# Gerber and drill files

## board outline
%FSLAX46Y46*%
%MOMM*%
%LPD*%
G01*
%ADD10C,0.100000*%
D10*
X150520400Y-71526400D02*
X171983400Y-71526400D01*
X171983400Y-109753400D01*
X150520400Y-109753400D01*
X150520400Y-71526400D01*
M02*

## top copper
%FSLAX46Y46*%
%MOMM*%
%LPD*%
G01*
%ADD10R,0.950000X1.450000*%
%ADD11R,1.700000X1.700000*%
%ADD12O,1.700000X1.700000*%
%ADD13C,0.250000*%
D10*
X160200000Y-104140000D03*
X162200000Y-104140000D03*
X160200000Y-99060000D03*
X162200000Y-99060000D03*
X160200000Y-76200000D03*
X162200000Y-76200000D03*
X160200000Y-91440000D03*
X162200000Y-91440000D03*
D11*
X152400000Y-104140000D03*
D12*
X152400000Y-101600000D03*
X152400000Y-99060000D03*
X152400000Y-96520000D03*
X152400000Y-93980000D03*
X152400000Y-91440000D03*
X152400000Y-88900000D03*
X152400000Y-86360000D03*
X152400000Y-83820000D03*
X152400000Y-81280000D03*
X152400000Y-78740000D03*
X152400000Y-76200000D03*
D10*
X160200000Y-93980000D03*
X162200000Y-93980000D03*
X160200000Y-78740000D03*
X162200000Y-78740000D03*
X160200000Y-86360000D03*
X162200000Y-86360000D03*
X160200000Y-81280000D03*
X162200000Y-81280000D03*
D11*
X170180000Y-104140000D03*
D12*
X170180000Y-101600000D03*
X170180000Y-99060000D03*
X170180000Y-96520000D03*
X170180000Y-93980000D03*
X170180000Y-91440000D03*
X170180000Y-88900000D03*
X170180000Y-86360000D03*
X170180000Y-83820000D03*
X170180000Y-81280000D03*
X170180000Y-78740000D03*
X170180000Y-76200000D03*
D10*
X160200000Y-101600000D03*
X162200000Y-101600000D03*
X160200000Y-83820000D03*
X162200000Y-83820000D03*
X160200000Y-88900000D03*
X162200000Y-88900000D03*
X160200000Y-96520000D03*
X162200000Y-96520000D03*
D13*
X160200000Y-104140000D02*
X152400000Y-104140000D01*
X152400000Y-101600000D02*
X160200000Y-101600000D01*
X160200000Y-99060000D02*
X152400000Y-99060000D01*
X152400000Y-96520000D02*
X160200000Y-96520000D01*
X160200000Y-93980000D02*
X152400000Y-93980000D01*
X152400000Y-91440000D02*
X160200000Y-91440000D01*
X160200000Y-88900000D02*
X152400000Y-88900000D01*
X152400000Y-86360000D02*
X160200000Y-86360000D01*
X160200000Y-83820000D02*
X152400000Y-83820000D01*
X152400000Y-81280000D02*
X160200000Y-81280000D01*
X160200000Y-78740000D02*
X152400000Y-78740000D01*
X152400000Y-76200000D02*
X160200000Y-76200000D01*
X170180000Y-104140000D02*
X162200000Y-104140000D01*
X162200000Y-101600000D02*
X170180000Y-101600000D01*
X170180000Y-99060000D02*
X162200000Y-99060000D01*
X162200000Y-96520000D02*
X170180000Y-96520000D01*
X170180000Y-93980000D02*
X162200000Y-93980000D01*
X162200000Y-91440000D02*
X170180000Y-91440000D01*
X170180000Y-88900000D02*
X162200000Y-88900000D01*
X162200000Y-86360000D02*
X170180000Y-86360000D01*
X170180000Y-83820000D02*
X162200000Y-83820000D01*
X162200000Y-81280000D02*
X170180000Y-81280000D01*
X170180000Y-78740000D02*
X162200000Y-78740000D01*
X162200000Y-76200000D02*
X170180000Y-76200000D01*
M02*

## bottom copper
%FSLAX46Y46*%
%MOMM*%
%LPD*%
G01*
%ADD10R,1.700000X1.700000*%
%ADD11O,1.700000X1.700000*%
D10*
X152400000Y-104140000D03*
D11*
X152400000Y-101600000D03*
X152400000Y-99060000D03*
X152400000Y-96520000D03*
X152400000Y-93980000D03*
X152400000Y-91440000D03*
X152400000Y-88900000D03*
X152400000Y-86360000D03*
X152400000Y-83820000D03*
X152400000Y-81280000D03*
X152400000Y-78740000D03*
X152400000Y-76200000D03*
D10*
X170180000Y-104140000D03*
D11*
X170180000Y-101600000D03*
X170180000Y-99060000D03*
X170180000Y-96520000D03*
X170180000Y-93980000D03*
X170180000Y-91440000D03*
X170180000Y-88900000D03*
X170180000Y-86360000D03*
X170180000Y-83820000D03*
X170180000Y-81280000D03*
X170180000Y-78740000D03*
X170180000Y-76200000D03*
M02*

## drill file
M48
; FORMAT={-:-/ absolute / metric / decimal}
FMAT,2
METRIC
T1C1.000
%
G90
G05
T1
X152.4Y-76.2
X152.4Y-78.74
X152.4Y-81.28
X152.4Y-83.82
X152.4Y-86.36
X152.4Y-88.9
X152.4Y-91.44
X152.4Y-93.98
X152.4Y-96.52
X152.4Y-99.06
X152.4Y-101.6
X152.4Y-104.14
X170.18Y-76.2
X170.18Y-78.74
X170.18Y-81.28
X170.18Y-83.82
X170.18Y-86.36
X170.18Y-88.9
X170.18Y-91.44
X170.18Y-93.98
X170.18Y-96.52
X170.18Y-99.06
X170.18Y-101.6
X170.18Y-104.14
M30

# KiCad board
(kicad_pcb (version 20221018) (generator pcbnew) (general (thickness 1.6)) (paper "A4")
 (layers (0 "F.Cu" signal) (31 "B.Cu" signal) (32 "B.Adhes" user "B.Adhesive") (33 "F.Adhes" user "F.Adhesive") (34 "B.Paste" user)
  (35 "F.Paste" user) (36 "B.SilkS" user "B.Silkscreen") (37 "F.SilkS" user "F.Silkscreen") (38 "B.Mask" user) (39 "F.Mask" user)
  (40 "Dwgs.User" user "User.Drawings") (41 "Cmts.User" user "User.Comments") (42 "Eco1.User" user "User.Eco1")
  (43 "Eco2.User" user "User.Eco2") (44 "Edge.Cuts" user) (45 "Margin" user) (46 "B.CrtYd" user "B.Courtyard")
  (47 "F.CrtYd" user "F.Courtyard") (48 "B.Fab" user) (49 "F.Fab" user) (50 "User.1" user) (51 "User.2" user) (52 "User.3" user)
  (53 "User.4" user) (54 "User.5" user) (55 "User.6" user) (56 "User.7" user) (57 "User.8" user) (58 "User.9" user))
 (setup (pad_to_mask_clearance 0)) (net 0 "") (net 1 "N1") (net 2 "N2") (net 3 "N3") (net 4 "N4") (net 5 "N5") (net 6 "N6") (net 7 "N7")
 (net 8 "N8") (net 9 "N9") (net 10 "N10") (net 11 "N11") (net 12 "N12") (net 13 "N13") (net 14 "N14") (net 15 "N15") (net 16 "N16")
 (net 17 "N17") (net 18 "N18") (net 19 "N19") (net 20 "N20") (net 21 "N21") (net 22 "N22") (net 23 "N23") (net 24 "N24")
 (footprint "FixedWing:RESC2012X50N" (layer "F.Cu") (at 161.2 104.14)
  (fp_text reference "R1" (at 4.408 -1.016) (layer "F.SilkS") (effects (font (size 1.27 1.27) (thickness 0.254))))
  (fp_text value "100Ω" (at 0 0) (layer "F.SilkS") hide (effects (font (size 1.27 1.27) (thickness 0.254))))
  (pad "1" smd rect (at -1 0) (size 0.95 1.45) (layers "F.Cu" "F.Paste" "F.Mask") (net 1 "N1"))
  (pad "2" smd rect (at 1 0) (size 0.95 1.45) (layers "F.Cu" "F.Paste" "F.Mask") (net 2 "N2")))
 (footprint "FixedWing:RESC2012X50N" (layer "F.Cu") (at 161.2 99.06)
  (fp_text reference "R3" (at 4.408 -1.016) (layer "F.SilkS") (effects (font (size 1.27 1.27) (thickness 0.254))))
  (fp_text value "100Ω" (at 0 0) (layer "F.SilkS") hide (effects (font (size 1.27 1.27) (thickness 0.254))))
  (pad "1" smd rect (at -1 0) (size 0.95 1.45) (layers "F.Cu" "F.Paste" "F.Mask") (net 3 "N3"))
  (pad "2" smd rect (at 1 0) (size 0.95 1.45) (layers "F.Cu" "F.Paste" "F.Mask") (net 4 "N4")))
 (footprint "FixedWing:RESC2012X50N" (layer "F.Cu") (at 161.2 76.2)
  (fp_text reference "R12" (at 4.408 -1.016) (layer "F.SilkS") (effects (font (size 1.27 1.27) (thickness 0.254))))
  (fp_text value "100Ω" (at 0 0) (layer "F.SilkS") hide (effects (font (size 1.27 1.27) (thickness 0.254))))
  (pad "1" smd rect (at -1 0) (size 0.95 1.45) (layers "F.Cu" "F.Paste" "F.Mask") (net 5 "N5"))
  (pad "2" smd rect (at 1 0) (size 0.95 1.45) (layers "F.Cu" "F.Paste" "F.Mask") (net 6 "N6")))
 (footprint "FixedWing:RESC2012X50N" (layer "F.Cu") (at 161.2 91.44)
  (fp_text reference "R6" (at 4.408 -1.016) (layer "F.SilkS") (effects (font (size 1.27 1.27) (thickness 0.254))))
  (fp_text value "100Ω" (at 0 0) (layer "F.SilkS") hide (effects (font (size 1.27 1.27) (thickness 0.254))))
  (pad "1" smd rect (at -1 0) (size 0.95 1.45) (layers "F.Cu" "F.Paste" "F.Mask") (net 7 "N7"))
  (pad "2" smd rect (at 1 0) (size 0.95 1.45) (layers "F.Cu" "F.Paste" "F.Mask") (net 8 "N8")))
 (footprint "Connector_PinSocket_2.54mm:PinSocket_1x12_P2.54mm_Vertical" (layer "F.Cu") (at 152.4 104.14 180)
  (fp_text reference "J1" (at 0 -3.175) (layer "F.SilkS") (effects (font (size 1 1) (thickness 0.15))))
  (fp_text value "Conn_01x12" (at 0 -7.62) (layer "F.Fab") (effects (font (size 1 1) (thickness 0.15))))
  (pad "1" thru_hole rect (at 0 0 180) (size 1.7 1.7) (drill 1) (layers "*.Cu" "*.Mask") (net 1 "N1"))
  (pad "2" thru_hole oval (at 0 2.54 180) (size 1.7 1.7) (drill 1) (layers "*.Cu" "*.Mask") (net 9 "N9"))
  (pad "3" thru_hole oval (at 0 5.08 180) (size 1.7 1.7) (drill 1) (layers "*.Cu" "*.Mask") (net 3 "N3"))
  (pad "4" thru_hole oval (at 0 7.62 180) (size 1.7 1.7) (drill 1) (layers "*.Cu" "*.Mask") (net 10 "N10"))
  (pad "5" thru_hole oval (at 0 10.16 180) (size 1.7 1.7) (drill 1) (layers "*.Cu" "*.Mask") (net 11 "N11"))
  (pad "6" thru_hole oval (at 0 12.7 180) (size 1.7 1.7) (drill 1) (layers "*.Cu" "*.Mask") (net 7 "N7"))
  (pad "7" thru_hole oval (at 0 15.24 180) (size 1.7 1.7) (drill 1) (layers "*.Cu" "*.Mask") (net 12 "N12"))
  (pad "8" thru_hole oval (at 0 17.78 180) (size 1.7 1.7) (drill 1) (layers "*.Cu" "*.Mask") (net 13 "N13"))
  (pad "9" thru_hole oval (at 0 20.32 180) (size 1.7 1.7) (drill 1) (layers "*.Cu" "*.Mask") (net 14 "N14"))
  (pad "10" thru_hole oval (at 0 22.86 180) (size 1.7 1.7) (drill 1) (layers "*.Cu" "*.Mask") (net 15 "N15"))
  (pad "11" thru_hole oval (at 0 25.4 180) (size 1.7 1.7) (drill 1) (layers "*.Cu" "*.Mask") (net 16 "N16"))
  (pad "12" thru_hole oval (at 0 27.94 180) (size 1.7 1.7) (drill 1) (layers "*.Cu" "*.Mask") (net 5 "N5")))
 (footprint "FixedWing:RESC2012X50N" (layer "F.Cu") (at 161.2 93.98)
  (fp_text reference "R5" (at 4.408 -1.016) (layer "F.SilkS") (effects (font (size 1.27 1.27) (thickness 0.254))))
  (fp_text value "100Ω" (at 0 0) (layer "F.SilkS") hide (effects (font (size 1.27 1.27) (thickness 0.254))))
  (pad "1" smd rect (at -1 0) (size 0.95 1.45) (layers "F.Cu" "F.Paste" "F.Mask") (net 11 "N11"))
  (pad "2" smd rect (at 1 0) (size 0.95 1.45) (layers "F.Cu" "F.Paste" "F.Mask") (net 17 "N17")))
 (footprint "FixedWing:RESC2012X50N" (layer "F.Cu") (at 161.2 78.74)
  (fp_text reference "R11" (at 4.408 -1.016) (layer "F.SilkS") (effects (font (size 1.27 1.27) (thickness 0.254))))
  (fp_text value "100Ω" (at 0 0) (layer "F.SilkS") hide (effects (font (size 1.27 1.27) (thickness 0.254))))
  (pad "1" smd rect (at -1 0) (size 0.95 1.45) (layers "F.Cu" "F.Paste" "F.Mask") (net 16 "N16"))
  (pad "2" smd rect (at 1 0) (size 0.95 1.45) (layers "F.Cu" "F.Paste" "F.Mask") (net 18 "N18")))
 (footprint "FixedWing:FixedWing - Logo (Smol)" (layer "F.Cu") (at 161.250214 73.970419)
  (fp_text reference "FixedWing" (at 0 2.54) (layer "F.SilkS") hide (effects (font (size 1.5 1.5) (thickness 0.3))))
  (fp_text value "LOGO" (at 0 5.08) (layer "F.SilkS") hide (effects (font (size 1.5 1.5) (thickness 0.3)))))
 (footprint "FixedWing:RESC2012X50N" (layer "F.Cu") (at 161.2 86.36)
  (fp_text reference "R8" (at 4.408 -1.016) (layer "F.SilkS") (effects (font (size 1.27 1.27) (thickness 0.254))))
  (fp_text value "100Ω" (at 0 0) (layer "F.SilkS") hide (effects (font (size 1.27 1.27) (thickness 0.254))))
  (pad "1" smd rect (at -1 0) (size 0.95 1.45) (layers "F.Cu" "F.Paste" "F.Mask") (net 13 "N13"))
  (pad "2" smd rect (at 1 0) (size 0.95 1.45) (layers "F.Cu" "F.Paste" "F.Mask") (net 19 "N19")))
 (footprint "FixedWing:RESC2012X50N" (layer "F.Cu") (at 161.2 81.28)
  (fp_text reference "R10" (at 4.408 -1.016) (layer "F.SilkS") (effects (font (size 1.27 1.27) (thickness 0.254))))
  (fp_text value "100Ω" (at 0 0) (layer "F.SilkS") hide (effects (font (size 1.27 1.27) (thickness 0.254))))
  (pad "1" smd rect (at -1 0) (size 0.95 1.45) (layers "F.Cu" "F.Paste" "F.Mask") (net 15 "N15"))
  (pad "2" smd rect (at 1 0) (size 0.95 1.45) (layers "F.Cu" "F.Paste" "F.Mask") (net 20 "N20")))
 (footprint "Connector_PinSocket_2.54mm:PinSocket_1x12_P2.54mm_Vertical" (layer "F.Cu") (at 170.18 104.14 180)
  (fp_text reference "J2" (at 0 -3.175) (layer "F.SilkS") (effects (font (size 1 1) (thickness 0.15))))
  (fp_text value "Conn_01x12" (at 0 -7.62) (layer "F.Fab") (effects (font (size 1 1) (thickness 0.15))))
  (pad "1" thru_hole rect (at 0 0 180) (size 1.7 1.7) (drill 1) (layers "*.Cu" "*.Mask") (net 2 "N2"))
  (pad "2" thru_hole oval (at 0 2.54 180) (size 1.7 1.7) (drill 1) (layers "*.Cu" "*.Mask") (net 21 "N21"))
  (pad "3" thru_hole oval (at 0 5.08 180) (size 1.7 1.7) (drill 1) (layers "*.Cu" "*.Mask") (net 4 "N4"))
  (pad "4" thru_hole oval (at 0 7.62 180) (size 1.7 1.7) (drill 1) (layers "*.Cu" "*.Mask") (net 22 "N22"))
  (pad "5" thru_hole oval (at 0 10.16 180) (size 1.7 1.7) (drill 1) (layers "*.Cu" "*.Mask") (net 17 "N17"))
  (pad "6" thru_hole oval (at 0 12.7 180) (size 1.7 1.7) (drill 1) (layers "*.Cu" "*.Mask") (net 8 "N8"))
  (pad "7" thru_hole oval (at 0 15.24 180) (size 1.7 1.7) (drill 1) (layers "*.Cu" "*.Mask") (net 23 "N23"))
  (pad "8" thru_hole oval (at 0 17.78 180) (size 1.7 1.7) (drill 1) (layers "*.Cu" "*.Mask") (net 19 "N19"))
  (pad "9" thru_hole oval (at 0 20.32 180) (size 1.7 1.7) (drill 1) (layers "*.Cu" "*.Mask") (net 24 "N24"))
  (pad "10" thru_hole oval (at 0 22.86 180) (size 1.7 1.7) (drill 1) (layers "*.Cu" "*.Mask") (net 20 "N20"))
  (pad "11" thru_hole oval (at 0 25.4 180) (size 1.7 1.7) (drill 1) (layers "*.Cu" "*.Mask") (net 18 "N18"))
  (pad "12" thru_hole oval (at 0 27.94 180) (size 1.7 1.7) (drill 1) (layers "*.Cu" "*.Mask") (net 6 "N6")))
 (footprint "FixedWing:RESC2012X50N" (layer "F.Cu") (at 161.2 101.6)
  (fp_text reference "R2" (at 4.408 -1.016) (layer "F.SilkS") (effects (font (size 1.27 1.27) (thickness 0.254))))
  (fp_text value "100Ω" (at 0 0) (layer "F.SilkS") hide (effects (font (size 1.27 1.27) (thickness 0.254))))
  (pad "1" smd rect (at -1 0) (size 0.95 1.45) (layers "F.Cu" "F.Paste" "F.Mask") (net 9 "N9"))
  (pad "2" smd rect (at 1 0) (size 0.95 1.45) (layers "F.Cu" "F.Paste" "F.Mask") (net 21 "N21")))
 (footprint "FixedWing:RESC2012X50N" (layer "F.Cu") (at 161.2 83.82)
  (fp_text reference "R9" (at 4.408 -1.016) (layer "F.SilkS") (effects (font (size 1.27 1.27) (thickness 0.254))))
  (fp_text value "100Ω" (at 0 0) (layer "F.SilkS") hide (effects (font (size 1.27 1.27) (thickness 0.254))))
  (pad "1" smd rect (at -1 0) (size 0.95 1.45) (layers "F.Cu" "F.Paste" "F.Mask") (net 14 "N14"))
  (pad "2" smd rect (at 1 0) (size 0.95 1.45) (layers "F.Cu" "F.Paste" "F.Mask") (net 24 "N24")))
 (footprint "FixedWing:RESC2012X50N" (layer "F.Cu") (at 161.2 88.9)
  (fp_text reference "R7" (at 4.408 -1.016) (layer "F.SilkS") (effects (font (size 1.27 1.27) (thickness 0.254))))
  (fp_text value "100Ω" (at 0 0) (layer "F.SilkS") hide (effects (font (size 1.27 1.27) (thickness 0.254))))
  (pad "1" smd rect (at -1 0) (size 0.95 1.45) (layers "F.Cu" "F.Paste" "F.Mask") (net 12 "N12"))
  (pad "2" smd rect (at 1 0) (size 0.95 1.45) (layers "F.Cu" "F.Paste" "F.Mask") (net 23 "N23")))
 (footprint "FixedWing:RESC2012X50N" (layer "F.Cu") (at 161.2 96.52)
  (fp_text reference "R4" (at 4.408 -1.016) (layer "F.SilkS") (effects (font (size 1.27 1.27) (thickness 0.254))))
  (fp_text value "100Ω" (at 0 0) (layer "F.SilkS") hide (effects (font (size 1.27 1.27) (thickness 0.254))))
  (pad "1" smd rect (at -1 0) (size 0.95 1.45) (layers "F.Cu" "F.Paste" "F.Mask") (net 10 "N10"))
  (pad "2" smd rect (at 1 0) (size 0.95 1.45) (layers "F.Cu" "F.Paste" "F.Mask") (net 22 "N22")))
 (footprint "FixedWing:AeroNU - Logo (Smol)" (layer "F.Cu") (at 161.355749 109.504388)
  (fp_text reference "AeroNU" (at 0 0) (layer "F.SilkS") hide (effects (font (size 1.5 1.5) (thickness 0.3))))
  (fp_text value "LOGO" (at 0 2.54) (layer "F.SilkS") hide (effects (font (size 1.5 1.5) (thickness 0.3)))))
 (gr_rect (start 150.5204 71.5264) (end 171.9834 109.7534) (stroke (width 0.1) (type default)) (fill none) (layer "Edge.Cuts"))
 (segment (start 160.2 104.14) (end 152.4 104.14) (width 0.25) (layer "F.Cu") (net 1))
 (segment (start 152.4 101.6) (end 160.2 101.6) (width 0.25) (layer "F.Cu") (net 9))
 (segment (start 160.2 99.06) (end 152.4 99.06) (width 0.25) (layer "F.Cu") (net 3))
 (segment (start 152.4 96.52) (end 160.2 96.52) (width 0.25) (layer "F.Cu") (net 10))
 (segment (start 160.2 93.98) (end 152.4 93.98) (width 0.25) (layer "F.Cu") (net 11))
 (segment (start 152.4 91.44) (end 160.2 91.44) (width 0.25) (layer "F.Cu") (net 7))
 (segment (start 160.2 88.9) (end 152.4 88.9) (width 0.25) (layer "F.Cu") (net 12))
 (segment (start 152.4 86.36) (end 160.2 86.36) (width 0.25) (layer "F.Cu") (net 13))
 (segment (start 160.2 83.82) (end 152.4 83.82) (width 0.25) (layer "F.Cu") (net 14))
 (segment (start 152.4 81.28) (end 160.2 81.28) (width 0.25) (layer "F.Cu") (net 15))
 (segment (start 160.2 78.74) (end 152.4 78.74) (width 0.25) (layer "F.Cu") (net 16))
 (segment (start 152.4 76.2) (end 160.2 76.2) (width 0.25) (layer "F.Cu") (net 5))
 (segment (start 170.18 104.14) (end 162.2 104.14) (width 0.25) (layer "F.Cu") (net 2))
 (segment (start 162.2 101.6) (end 170.18 101.6) (width 0.25) (layer "F.Cu") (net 21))
 (segment (start 170.18 99.06) (end 162.2 99.06) (width 0.25) (layer "F.Cu") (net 4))
 (segment (start 162.2 96.52) (end 170.18 96.52) (width 0.25) (layer "F.Cu") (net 22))
 (segment (start 170.18 93.98) (end 162.2 93.98) (width 0.25) (layer "F.Cu") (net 17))
 (segment (start 162.2 91.44) (end 170.18 91.44) (width 0.25) (layer "F.Cu") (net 8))
 (segment (start 170.18 88.9) (end 162.2 88.9) (width 0.25) (layer "F.Cu") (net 23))
 (segment (start 162.2 86.36) (end 170.18 86.36) (width 0.25) (layer "F.Cu") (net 19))
 (segment (start 170.18 83.82) (end 162.2 83.82) (width 0.25) (layer "F.Cu") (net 24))
 (segment (start 162.2 81.28) (end 170.18 81.28) (width 0.25) (layer "F.Cu") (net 20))
 (segment (start 170.18 78.74) (end 162.2 78.74) (width 0.25) (layer "F.Cu") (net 18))
 (segment (start 162.2 76.2) (end 170.18 76.2) (width 0.25) (layer "F.Cu") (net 6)))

